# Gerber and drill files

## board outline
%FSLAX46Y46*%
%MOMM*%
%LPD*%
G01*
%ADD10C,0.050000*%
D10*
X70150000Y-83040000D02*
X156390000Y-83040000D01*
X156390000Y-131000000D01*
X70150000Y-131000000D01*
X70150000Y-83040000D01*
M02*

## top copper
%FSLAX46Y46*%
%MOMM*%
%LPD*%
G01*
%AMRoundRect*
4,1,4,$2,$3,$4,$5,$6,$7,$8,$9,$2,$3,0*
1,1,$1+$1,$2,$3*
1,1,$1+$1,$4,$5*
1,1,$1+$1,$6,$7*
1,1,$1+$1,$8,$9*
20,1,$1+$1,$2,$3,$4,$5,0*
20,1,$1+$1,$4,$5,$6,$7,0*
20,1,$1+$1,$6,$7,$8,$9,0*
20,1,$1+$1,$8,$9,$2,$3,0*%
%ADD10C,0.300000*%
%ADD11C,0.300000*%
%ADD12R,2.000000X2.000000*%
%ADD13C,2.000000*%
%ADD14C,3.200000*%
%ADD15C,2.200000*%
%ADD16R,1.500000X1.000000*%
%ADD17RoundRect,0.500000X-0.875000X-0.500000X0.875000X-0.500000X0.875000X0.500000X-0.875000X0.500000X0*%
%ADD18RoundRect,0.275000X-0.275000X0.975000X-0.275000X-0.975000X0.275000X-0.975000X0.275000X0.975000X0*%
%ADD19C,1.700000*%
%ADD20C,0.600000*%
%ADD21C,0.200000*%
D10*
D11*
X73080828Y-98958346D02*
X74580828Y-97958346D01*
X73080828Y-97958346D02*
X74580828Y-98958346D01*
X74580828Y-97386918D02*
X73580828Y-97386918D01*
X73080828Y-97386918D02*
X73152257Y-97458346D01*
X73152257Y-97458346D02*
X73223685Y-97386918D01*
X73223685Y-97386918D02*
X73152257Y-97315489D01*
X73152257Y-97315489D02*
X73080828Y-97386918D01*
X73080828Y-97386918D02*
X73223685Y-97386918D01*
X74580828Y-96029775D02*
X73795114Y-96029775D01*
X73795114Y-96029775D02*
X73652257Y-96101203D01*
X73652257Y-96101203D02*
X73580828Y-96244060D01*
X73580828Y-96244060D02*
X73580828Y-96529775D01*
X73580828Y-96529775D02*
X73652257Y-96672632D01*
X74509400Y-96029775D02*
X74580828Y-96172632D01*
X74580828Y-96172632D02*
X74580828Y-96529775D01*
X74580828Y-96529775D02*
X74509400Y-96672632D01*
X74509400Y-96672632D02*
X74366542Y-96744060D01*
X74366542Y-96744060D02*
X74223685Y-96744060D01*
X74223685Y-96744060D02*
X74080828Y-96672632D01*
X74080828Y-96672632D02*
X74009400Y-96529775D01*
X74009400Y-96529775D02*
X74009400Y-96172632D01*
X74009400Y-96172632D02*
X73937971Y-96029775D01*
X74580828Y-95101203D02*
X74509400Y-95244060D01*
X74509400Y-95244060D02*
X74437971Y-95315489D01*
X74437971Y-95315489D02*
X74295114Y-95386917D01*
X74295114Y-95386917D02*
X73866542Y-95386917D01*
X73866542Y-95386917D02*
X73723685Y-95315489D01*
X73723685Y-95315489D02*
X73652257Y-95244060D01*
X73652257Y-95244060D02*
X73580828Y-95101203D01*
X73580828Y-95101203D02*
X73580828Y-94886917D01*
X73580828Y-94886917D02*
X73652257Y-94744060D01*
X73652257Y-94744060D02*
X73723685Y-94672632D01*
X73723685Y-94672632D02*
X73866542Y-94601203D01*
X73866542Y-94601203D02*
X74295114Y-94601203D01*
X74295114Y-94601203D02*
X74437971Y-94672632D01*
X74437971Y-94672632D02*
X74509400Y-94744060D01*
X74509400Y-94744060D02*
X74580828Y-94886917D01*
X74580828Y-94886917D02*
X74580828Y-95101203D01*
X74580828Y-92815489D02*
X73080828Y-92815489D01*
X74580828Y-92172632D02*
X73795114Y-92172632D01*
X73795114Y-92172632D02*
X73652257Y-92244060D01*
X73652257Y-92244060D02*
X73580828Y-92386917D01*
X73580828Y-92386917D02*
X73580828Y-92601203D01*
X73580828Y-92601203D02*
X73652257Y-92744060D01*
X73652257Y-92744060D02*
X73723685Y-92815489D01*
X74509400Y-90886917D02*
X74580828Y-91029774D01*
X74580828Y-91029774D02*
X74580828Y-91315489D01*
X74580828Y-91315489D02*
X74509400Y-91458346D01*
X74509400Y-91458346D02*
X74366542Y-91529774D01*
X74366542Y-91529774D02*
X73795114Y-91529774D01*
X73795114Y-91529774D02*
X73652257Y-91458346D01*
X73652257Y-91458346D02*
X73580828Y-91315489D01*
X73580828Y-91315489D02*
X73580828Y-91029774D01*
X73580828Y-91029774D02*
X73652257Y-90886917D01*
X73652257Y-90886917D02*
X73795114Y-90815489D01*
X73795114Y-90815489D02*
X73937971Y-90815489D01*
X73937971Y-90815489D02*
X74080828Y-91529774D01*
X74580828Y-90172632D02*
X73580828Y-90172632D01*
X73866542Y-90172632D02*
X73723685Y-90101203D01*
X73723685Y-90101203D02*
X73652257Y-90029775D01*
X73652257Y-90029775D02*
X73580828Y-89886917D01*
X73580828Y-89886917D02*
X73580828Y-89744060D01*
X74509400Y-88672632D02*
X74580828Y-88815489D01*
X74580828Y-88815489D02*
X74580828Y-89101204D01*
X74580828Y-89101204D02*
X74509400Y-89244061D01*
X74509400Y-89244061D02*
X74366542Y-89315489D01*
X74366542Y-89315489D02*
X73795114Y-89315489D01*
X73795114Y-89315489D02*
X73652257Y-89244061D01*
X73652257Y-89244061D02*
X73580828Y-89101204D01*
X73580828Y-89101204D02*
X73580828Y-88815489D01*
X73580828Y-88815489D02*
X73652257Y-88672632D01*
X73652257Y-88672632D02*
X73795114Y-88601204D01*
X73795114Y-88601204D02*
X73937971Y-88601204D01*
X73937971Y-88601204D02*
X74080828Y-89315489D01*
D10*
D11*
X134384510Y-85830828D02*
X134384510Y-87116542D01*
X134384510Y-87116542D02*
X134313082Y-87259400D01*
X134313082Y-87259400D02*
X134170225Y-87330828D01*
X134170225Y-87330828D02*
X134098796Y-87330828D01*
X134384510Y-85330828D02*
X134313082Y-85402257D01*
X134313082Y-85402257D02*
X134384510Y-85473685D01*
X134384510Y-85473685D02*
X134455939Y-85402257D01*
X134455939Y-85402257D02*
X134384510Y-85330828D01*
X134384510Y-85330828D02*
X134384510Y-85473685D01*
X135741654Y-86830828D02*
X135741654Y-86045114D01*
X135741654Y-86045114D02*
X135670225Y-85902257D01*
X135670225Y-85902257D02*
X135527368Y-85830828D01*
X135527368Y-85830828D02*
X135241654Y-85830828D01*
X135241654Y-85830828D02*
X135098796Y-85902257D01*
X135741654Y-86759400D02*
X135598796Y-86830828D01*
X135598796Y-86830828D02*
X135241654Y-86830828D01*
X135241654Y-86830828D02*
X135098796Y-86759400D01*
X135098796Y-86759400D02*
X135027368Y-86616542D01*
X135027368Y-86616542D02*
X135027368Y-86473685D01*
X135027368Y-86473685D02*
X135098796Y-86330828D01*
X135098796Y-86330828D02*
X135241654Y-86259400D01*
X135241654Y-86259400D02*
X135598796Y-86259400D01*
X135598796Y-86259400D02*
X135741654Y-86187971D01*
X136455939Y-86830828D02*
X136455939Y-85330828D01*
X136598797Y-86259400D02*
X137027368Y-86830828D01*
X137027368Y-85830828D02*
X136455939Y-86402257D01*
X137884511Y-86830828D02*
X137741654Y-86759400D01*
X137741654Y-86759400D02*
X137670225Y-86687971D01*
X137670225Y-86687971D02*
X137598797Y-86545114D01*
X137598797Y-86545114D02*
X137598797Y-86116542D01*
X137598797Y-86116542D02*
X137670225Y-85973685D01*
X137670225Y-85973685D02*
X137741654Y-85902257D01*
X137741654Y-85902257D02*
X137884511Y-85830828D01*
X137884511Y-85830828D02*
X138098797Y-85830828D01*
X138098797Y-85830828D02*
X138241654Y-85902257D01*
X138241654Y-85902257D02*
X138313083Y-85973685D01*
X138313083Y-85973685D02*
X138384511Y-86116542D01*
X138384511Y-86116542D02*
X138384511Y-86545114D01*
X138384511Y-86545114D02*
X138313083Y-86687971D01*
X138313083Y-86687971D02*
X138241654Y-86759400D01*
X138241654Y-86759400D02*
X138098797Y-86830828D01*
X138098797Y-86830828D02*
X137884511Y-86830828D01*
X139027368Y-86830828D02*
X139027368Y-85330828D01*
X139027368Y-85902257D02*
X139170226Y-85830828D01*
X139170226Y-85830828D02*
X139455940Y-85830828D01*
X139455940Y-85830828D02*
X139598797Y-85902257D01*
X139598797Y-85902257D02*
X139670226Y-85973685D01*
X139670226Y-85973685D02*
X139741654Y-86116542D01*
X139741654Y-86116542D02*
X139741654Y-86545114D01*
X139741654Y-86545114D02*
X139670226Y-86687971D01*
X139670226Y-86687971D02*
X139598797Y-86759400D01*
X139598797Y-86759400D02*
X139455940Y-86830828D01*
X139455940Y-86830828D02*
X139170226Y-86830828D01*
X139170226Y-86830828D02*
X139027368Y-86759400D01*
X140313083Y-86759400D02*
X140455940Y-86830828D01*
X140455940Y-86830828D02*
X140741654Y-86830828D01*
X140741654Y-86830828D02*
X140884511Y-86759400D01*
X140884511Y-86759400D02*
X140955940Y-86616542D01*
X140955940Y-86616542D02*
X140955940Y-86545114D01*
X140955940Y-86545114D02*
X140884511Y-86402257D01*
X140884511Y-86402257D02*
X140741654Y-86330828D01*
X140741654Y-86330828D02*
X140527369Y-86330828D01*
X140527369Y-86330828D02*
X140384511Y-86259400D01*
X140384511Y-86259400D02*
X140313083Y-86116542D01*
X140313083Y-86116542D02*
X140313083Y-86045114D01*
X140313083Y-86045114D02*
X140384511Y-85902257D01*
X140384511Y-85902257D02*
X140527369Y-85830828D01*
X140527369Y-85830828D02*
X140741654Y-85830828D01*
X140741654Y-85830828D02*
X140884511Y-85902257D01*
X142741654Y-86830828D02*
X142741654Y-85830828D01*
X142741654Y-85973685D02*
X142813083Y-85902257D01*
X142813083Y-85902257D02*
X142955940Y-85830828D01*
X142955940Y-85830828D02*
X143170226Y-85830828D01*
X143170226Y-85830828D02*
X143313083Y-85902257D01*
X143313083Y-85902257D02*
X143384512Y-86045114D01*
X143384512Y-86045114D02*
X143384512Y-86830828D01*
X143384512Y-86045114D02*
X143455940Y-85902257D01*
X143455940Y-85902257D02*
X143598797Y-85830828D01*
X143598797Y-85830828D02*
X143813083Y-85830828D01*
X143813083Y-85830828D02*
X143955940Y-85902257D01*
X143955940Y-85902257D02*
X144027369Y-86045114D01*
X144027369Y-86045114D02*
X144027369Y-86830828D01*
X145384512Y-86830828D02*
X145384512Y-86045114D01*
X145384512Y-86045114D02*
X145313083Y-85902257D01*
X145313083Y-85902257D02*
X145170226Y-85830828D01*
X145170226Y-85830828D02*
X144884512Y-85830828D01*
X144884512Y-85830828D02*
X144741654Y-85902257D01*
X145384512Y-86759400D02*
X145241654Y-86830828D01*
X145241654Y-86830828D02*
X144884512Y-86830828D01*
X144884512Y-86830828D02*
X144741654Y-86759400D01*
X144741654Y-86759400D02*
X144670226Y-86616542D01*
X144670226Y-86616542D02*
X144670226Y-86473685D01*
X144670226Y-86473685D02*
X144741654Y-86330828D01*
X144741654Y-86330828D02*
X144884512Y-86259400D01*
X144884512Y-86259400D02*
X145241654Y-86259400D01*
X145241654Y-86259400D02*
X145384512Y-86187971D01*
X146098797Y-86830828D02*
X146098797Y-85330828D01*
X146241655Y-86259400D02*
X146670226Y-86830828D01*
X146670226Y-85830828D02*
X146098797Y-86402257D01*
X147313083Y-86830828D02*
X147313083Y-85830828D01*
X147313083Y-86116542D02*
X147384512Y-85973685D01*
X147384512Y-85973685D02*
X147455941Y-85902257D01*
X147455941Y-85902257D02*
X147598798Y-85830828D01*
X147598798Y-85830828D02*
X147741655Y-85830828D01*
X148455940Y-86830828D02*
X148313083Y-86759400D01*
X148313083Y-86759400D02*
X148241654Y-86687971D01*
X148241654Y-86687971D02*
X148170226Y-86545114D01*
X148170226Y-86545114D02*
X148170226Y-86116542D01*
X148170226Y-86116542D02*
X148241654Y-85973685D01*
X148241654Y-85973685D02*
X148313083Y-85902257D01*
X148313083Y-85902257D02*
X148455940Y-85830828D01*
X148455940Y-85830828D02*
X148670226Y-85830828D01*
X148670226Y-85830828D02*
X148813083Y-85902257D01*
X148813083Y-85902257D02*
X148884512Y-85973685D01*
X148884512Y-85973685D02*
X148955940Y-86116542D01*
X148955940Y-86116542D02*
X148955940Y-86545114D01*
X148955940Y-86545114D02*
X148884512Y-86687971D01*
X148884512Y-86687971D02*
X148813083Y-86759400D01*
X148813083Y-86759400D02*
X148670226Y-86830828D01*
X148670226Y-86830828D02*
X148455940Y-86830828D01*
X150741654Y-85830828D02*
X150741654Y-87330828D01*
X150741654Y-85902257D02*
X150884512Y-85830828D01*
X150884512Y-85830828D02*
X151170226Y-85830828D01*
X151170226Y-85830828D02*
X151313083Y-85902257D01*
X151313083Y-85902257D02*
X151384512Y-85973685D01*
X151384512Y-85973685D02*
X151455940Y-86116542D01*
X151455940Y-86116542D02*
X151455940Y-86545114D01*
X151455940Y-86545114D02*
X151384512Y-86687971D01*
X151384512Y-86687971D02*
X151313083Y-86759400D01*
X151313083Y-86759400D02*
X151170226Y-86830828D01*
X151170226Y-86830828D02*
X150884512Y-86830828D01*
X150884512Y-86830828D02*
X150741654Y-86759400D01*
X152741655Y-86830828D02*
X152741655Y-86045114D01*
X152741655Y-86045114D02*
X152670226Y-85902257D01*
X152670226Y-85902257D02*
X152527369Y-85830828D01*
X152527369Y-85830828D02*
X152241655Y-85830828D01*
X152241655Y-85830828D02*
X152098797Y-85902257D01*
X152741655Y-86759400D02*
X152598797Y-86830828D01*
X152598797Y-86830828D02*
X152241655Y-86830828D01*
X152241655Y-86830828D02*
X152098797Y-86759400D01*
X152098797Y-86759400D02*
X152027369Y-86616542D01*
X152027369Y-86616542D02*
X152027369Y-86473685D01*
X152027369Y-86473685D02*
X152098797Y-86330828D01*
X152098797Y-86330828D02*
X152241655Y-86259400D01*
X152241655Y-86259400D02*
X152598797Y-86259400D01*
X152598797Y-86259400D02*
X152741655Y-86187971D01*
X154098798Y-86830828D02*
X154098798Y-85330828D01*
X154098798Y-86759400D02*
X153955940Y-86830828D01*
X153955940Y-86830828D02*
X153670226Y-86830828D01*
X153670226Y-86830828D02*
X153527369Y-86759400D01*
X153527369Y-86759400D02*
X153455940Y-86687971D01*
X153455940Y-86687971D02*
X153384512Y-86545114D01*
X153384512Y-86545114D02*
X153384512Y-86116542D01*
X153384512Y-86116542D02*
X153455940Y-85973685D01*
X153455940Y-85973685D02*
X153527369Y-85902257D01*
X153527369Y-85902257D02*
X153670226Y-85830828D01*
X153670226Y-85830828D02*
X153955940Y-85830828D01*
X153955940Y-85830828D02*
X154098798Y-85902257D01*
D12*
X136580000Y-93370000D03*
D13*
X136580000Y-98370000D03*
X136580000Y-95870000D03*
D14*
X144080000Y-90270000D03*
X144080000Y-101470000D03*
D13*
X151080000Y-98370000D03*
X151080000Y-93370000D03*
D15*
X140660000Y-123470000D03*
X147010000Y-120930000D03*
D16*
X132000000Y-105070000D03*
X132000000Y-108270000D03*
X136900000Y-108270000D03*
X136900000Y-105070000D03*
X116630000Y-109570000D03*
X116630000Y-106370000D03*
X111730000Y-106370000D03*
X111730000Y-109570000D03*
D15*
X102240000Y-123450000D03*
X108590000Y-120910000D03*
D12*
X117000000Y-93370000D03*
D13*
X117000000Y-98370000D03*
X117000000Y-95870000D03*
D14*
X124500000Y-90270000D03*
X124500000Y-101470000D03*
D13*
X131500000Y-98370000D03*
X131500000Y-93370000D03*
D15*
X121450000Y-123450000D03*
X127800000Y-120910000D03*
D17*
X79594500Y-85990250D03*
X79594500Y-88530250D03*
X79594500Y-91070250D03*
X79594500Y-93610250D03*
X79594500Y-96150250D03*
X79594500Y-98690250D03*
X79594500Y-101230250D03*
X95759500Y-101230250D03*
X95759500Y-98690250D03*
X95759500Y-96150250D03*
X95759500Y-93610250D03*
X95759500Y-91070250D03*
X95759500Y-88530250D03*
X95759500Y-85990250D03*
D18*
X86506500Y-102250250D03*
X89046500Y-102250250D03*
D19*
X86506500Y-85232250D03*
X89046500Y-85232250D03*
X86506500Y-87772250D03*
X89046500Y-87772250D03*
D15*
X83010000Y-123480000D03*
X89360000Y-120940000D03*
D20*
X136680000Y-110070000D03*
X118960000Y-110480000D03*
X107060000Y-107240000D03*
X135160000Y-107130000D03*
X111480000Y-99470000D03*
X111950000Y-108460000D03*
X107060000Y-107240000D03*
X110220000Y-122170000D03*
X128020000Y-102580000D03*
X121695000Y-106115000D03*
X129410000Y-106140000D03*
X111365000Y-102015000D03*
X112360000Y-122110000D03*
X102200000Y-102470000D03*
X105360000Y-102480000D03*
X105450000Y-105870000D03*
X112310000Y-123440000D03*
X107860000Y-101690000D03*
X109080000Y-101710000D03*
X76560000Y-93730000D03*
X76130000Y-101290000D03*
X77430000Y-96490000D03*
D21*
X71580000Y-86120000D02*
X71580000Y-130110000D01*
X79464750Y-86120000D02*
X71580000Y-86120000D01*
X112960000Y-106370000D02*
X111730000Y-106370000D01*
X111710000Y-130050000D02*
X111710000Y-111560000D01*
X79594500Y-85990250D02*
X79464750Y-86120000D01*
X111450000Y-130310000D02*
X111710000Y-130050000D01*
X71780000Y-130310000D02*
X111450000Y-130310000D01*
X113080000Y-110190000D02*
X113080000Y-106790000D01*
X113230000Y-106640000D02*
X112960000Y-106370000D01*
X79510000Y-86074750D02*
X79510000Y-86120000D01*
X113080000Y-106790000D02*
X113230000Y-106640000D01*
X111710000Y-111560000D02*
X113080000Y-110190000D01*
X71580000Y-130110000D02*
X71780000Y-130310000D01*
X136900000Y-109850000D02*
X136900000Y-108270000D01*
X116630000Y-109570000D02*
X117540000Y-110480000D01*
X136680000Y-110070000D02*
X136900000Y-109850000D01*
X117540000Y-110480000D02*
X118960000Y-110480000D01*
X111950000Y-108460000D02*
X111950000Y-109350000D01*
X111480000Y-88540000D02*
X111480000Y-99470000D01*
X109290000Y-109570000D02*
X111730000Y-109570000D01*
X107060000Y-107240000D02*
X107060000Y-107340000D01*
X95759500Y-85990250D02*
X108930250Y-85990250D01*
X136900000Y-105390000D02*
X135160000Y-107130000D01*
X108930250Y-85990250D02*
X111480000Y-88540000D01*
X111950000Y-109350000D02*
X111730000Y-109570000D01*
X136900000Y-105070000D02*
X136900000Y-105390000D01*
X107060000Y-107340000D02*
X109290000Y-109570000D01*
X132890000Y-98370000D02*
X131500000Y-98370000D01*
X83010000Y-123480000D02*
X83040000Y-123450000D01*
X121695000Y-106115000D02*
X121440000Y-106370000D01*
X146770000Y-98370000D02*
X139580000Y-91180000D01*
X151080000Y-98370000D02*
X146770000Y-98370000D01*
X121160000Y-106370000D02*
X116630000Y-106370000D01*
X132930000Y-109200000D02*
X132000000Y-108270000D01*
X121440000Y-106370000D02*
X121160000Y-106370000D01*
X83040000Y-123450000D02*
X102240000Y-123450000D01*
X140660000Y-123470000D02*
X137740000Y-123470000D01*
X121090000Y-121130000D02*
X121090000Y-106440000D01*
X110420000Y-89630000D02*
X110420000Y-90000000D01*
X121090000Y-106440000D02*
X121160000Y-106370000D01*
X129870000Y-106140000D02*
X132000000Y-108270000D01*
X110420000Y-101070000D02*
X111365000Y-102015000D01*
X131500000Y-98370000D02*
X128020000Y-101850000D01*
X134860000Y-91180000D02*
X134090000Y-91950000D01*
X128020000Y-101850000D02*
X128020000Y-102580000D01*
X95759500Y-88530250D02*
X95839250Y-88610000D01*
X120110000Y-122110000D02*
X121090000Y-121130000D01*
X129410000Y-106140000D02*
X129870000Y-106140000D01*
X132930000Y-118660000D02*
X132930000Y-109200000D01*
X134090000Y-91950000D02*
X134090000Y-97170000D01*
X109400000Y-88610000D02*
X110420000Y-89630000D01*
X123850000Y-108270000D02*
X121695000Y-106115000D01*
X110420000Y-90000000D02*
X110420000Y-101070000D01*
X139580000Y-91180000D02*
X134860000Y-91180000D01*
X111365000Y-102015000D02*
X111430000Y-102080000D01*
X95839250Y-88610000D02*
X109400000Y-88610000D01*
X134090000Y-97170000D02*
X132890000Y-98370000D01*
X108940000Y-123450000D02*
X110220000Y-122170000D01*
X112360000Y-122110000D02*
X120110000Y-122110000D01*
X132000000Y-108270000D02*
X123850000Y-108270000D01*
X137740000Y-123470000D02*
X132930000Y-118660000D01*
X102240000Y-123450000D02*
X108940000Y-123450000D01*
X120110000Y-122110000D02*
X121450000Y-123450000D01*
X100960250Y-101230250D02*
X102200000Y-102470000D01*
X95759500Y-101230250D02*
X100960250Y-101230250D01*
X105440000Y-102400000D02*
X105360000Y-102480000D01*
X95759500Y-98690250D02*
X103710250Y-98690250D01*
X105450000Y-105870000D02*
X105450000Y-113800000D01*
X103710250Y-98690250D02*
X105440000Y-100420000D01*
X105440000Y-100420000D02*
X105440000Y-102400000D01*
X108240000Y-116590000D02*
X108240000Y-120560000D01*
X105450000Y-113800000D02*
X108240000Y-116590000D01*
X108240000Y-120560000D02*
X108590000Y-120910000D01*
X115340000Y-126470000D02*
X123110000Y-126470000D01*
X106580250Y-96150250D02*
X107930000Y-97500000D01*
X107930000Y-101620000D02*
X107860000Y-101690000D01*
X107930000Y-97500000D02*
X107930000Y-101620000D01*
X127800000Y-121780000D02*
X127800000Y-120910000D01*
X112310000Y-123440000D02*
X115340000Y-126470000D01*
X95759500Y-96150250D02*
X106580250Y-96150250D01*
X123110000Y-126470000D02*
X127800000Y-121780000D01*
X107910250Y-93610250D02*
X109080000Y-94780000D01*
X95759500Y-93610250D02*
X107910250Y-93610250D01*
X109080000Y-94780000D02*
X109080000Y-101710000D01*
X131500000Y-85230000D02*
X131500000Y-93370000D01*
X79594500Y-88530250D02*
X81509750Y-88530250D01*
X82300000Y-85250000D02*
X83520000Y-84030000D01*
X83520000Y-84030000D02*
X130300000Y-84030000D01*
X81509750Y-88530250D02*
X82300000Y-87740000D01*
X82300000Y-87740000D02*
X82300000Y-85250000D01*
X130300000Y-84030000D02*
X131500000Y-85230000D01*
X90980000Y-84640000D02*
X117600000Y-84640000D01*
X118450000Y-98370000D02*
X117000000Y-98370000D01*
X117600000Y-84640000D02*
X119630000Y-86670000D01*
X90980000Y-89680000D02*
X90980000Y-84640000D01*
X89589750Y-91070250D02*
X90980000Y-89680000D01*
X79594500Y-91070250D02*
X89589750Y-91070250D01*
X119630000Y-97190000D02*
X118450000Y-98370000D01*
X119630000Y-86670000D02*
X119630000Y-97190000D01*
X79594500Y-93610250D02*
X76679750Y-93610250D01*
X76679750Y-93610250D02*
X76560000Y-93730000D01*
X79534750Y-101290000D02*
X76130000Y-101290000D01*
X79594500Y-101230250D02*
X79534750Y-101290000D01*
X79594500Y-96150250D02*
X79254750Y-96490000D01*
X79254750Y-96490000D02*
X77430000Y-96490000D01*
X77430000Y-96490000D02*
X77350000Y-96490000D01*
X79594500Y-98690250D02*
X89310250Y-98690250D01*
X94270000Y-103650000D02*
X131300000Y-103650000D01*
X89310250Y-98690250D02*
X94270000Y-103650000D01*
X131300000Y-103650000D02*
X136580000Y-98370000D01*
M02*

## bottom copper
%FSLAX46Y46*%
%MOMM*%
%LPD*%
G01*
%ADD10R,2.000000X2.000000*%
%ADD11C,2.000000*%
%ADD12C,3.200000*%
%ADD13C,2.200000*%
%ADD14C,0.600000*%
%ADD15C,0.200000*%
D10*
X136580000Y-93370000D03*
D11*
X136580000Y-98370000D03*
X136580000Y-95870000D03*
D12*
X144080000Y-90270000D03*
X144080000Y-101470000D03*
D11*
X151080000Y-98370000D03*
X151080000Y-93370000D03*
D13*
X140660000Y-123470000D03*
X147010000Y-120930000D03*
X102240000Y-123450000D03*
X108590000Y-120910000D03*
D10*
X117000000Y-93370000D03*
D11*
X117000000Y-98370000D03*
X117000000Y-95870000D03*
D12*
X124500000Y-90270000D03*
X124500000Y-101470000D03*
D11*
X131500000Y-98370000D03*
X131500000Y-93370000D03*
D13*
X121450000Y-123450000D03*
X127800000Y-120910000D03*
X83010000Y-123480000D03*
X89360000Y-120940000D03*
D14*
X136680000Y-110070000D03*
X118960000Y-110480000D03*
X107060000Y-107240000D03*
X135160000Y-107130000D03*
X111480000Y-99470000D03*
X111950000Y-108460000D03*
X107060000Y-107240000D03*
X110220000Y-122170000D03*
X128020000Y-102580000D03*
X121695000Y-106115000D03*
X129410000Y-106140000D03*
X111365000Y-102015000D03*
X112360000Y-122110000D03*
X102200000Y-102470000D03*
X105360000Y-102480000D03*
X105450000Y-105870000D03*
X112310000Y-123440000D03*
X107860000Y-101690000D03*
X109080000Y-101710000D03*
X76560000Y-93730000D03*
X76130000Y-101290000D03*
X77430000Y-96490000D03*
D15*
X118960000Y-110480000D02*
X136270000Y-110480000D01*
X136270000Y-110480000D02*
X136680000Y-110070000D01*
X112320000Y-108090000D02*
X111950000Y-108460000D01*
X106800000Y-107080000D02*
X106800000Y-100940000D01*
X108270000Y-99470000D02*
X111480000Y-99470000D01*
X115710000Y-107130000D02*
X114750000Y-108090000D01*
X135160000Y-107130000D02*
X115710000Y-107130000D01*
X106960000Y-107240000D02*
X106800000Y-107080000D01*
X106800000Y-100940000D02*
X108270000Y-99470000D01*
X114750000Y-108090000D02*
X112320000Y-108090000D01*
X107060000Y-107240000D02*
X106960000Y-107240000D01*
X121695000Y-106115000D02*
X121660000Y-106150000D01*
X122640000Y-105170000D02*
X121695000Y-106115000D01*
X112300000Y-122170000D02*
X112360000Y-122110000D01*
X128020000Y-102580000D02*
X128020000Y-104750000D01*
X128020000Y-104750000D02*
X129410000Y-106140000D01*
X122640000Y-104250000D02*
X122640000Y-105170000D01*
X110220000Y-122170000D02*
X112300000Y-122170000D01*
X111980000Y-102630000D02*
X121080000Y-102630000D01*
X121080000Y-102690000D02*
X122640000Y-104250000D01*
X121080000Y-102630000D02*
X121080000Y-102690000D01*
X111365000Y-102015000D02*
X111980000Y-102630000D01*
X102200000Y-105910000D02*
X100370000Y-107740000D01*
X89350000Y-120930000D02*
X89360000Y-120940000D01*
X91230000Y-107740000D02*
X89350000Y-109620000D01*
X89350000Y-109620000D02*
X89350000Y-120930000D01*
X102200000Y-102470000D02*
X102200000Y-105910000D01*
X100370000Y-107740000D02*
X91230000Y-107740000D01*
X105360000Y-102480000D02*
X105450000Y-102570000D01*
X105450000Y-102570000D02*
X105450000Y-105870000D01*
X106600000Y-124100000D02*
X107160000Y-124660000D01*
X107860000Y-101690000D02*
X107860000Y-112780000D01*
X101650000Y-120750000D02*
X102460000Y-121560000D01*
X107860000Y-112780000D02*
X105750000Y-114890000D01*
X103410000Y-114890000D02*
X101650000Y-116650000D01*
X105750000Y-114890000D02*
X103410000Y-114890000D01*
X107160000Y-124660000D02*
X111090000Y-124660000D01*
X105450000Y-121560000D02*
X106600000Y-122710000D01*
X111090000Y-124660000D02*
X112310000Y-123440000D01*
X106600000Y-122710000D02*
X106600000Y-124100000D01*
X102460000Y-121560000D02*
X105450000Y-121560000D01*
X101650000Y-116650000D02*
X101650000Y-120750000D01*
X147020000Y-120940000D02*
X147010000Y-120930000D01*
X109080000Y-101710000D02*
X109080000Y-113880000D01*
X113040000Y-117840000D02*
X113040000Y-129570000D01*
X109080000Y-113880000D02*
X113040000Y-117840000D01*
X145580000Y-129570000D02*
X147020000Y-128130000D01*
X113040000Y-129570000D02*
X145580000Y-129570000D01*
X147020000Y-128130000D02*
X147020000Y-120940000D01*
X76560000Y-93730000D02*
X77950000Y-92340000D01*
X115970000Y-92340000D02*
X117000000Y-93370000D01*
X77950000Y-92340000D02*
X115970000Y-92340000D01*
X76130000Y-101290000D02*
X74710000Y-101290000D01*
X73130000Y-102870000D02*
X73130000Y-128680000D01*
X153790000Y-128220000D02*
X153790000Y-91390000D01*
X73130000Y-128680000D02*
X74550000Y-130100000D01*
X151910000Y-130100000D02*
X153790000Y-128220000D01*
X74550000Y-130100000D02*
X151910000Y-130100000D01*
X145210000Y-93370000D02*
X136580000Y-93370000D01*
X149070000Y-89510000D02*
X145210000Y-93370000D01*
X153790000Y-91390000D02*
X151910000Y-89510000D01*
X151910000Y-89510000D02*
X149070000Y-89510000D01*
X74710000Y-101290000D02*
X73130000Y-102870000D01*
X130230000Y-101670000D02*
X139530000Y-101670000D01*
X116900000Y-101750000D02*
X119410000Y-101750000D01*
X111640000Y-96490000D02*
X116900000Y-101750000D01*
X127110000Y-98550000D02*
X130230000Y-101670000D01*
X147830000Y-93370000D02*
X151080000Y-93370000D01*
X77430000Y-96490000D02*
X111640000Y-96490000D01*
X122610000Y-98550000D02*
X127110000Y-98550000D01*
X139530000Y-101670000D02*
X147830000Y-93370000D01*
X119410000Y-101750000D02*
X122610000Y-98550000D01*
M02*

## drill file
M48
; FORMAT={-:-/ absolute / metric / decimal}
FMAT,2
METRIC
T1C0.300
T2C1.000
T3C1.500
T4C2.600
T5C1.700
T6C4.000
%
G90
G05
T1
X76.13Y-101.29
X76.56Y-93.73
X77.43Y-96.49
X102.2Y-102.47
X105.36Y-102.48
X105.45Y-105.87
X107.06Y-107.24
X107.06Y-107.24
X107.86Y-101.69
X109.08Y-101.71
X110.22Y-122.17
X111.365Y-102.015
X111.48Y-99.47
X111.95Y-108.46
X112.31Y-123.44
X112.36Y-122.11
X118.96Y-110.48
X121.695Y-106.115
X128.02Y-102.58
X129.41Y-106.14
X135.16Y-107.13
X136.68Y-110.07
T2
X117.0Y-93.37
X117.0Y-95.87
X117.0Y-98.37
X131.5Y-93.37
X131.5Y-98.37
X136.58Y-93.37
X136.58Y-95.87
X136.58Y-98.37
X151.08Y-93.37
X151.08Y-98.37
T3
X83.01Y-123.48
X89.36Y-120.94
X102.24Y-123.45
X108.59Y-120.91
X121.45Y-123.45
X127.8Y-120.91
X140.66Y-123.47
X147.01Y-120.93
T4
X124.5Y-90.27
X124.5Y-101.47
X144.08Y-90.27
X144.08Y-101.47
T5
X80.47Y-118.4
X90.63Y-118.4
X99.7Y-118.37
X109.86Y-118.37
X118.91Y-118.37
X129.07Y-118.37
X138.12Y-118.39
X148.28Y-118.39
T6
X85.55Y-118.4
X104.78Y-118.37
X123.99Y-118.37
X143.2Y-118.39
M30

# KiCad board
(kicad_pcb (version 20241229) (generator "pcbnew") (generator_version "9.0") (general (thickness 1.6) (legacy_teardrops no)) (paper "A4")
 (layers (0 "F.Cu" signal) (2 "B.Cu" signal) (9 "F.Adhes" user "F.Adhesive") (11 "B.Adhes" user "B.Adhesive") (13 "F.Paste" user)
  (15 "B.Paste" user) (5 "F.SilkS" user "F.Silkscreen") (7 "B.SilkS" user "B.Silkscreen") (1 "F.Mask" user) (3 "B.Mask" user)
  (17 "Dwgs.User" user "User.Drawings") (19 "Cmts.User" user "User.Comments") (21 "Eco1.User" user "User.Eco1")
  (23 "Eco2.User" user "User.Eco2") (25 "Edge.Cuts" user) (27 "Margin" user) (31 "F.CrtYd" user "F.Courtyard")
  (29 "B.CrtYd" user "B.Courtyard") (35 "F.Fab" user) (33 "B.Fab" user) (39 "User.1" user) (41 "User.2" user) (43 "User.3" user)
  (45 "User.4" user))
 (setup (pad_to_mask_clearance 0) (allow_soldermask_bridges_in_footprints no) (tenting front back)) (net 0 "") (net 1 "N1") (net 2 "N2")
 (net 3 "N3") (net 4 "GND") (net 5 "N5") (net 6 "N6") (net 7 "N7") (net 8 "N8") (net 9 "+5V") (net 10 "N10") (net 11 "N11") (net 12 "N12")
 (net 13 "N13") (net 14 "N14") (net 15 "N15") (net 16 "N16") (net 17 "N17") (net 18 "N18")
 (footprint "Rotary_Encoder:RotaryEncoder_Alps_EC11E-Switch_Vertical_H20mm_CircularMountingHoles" (layer "F.Cu") (at 136.58 93.37)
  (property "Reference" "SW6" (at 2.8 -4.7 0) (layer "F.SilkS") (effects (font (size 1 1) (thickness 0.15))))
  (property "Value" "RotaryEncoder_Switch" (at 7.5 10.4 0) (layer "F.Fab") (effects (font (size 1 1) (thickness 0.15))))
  (pad "A" thru_hole rect (at 0 0) (size 2 2) (drill 1) (layers "*.Cu" "*.Mask") (remove_unused_layers no) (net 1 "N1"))
  (pad "B" thru_hole circle (at 0 5) (size 2 2) (drill 1) (layers "*.Cu" "*.Mask") (remove_unused_layers no) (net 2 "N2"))
  (pad "C" thru_hole circle (at 0 2.5) (size 2 2) (drill 1) (layers "*.Cu" "*.Mask") (remove_unused_layers no) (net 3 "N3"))
  (pad "MP" thru_hole circle (at 7.5 -3.1) (size 3.2 3.2) (drill 2.6) (layers "*.Cu" "*.Mask") (remove_unused_layers no))
  (pad "MP" thru_hole circle (at 7.5 8.1) (size 3.2 3.2) (drill 2.6) (layers "*.Cu" "*.Mask") (remove_unused_layers no))
  (pad "S1" thru_hole circle (at 14.5 5) (size 2 2) (drill 1) (layers "*.Cu" "*.Mask") (remove_unused_layers no) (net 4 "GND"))
  (pad "S2" thru_hole circle (at 14.5 0) (size 2 2) (drill 1) (layers "*.Cu" "*.Mask") (remove_unused_layers no) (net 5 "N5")))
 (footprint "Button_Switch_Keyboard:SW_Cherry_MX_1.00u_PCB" (layer "F.Cu") (at 140.66 123.47 180)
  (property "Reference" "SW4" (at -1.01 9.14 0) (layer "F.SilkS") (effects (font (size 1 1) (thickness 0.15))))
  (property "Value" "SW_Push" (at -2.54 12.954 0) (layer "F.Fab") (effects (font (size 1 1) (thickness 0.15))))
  (pad "" np_thru_hole circle (at -7.62 5.08 180) (size 1.7 1.7) (drill 1.7) (layers "*.Cu" "*.Mask"))
  (pad "" np_thru_hole circle (at -2.54 5.08 180) (size 4 4) (drill 4) (layers "*.Cu" "*.Mask"))
  (pad "" np_thru_hole circle (at 2.54 5.08 180) (size 1.7 1.7) (drill 1.7) (layers "*.Cu" "*.Mask"))
  (pad "1" thru_hole circle (at 0 0 180) (size 2.2 2.2) (drill 1.5) (layers "*.Cu" "*.Mask") (remove_unused_layers no) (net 4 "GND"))
  (pad "2" thru_hole circle (at -6.35 2.54 180) (size 2.2 2.2) (drill 1.5) (layers "*.Cu" "*.Mask") (remove_unused_layers no) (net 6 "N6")))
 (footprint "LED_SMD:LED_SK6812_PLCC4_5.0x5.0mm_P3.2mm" (layer "F.Cu") (at 134.45 106.67)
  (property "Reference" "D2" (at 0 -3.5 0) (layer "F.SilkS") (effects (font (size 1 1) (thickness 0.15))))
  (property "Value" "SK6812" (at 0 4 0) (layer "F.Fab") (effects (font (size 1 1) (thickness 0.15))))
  (pad "1" smd rect (at -2.45 -1.6 180) (size 1.5 1) (layers "F.Cu" "F.Mask" "F.Paste") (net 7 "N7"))
  (pad "2" smd rect (at -2.45 1.6 180) (size 1.5 1) (layers "F.Cu" "F.Mask" "F.Paste") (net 4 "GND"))
  (pad "3" smd rect (at 2.45 1.6 180) (size 1.5 1) (layers "F.Cu" "F.Mask" "F.Paste") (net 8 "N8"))
  (pad "4" smd rect (at 2.45 -1.6 180) (size 1.5 1) (layers "F.Cu" "F.Mask" "F.Paste") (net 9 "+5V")))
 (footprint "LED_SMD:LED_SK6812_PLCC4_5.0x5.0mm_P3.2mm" (layer "F.Cu") (at 114.18 107.97 180)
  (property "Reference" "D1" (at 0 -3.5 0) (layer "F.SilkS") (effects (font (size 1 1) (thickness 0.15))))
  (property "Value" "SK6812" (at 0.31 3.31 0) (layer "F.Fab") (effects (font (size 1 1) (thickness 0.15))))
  (pad "1" smd rect (at -2.45 -1.6) (size 1.5 1) (layers "F.Cu" "F.Mask" "F.Paste") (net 8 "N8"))
  (pad "2" smd rect (at -2.45 1.6) (size 1.5 1) (layers "F.Cu" "F.Mask" "F.Paste") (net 4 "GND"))
  (pad "3" smd rect (at 2.45 1.6) (size 1.5 1) (layers "F.Cu" "F.Mask" "F.Paste") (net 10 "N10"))
  (pad "4" smd rect (at 2.45 -1.6) (size 1.5 1) (layers "F.Cu" "F.Mask" "F.Paste") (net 9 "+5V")))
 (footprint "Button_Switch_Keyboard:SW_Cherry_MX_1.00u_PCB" (layer "F.Cu") (at 102.24 123.45 180)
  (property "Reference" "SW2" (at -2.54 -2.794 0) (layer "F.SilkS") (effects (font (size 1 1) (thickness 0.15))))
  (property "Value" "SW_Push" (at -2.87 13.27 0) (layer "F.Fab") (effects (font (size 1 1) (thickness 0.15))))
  (pad "" np_thru_hole circle (at -7.62 5.08 180) (size 1.7 1.7) (drill 1.7) (layers "*.Cu" "*.Mask"))
  (pad "" np_thru_hole circle (at -2.54 5.08 180) (size 4 4) (drill 4) (layers "*.Cu" "*.Mask"))
  (pad "" np_thru_hole circle (at 2.54 5.08 180) (size 1.7 1.7) (drill 1.7) (layers "*.Cu" "*.Mask"))
  (pad "1" thru_hole circle (at 0 0 180) (size 2.2 2.2) (drill 1.5) (layers "*.Cu" "*.Mask") (remove_unused_layers no) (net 4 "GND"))
  (pad "2" thru_hole circle (at -6.35 2.54 180) (size 2.2 2.2) (drill 1.5) (layers "*.Cu" "*.Mask") (remove_unused_layers no) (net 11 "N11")))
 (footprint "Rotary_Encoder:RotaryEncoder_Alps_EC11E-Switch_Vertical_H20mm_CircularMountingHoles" (layer "F.Cu") (at 117 93.37)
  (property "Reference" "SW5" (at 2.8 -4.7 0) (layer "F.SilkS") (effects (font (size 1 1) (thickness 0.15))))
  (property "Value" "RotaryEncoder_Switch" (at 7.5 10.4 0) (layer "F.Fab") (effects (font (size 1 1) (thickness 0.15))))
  (pad "A" thru_hole rect (at 0 0) (size 2 2) (drill 1) (layers "*.Cu" "*.Mask") (remove_unused_layers no) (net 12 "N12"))
  (pad "B" thru_hole circle (at 0 5) (size 2 2) (drill 1) (layers "*.Cu" "*.Mask") (remove_unused_layers no) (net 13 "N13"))
  (pad "C" thru_hole circle (at 0 2.5) (size 2 2) (drill 1) (layers "*.Cu" "*.Mask") (remove_unused_layers no) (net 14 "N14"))
  (pad "MP" thru_hole circle (at 7.5 -3.1) (size 3.2 3.2) (drill 2.6) (layers "*.Cu" "*.Mask") (remove_unused_layers no))
  (pad "MP" thru_hole circle (at 7.5 8.1) (size 3.2 3.2) (drill 2.6) (layers "*.Cu" "*.Mask") (remove_unused_layers no))
  (pad "S1" thru_hole circle (at 14.5 5) (size 2 2) (drill 1) (layers "*.Cu" "*.Mask") (remove_unused_layers no) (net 4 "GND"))
  (pad "S2" thru_hole circle (at 14.5 0) (size 2 2) (drill 1) (layers "*.Cu" "*.Mask") (remove_unused_layers no) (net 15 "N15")))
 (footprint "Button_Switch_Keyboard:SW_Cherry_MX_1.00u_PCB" (layer "F.Cu") (at 121.45 123.45 180)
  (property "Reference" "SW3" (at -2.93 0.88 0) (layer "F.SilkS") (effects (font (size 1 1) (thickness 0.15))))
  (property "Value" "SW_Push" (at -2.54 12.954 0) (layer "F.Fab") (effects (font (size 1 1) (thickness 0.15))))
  (pad "" np_thru_hole circle (at -7.62 5.08 180) (size 1.7 1.7) (drill 1.7) (layers "*.Cu" "*.Mask"))
  (pad "" np_thru_hole circle (at -2.54 5.08 180) (size 4 4) (drill 4) (layers "*.Cu" "*.Mask"))
  (pad "" np_thru_hole circle (at 2.54 5.08 180) (size 1.7 1.7) (drill 1.7) (layers "*.Cu" "*.Mask"))
  (pad "1" thru_hole circle (at 0 0 180) (size 2.2 2.2) (drill 1.5) (layers "*.Cu" "*.Mask") (remove_unused_layers no) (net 4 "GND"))
  (pad "2" thru_hole circle (at -6.35 2.54 180) (size 2.2 2.2) (drill 1.5) (layers "*.Cu" "*.Mask") (remove_unused_layers no) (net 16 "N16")))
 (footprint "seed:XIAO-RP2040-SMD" (layer "F.Cu") (at 87.5945 93.61025)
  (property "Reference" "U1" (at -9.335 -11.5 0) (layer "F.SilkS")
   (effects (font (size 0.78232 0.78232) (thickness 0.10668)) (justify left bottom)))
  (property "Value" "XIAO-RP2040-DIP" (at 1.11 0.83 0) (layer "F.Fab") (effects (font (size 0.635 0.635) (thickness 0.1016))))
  (pad "1" smd roundrect (at -8 -7.62) (size 2.75 2) (layers "F.Cu" "F.Mask" "F.Paste") (roundrect_rratio 0.25) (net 10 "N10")
   (solder_mask_margin 0.0508) (thermal_bridge_angle 45))
  (pad "2" smd roundrect (at -8 -5.08) (size 2.75 2) (layers "F.Cu" "F.Mask" "F.Paste") (roundrect_rratio 0.25) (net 15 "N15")
   (solder_mask_margin 0.0508) (thermal_bridge_angle 45))
  (pad "3" smd roundrect (at -8 -2.54) (size 2.75 2) (layers "F.Cu" "F.Mask" "F.Paste") (roundrect_rratio 0.25) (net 13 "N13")
   (solder_mask_margin 0.0508) (thermal_bridge_angle 45))
  (pad "4" smd roundrect (at -8 0) (size 2.75 2) (layers "F.Cu" "F.Mask" "F.Paste") (roundrect_rratio 0.25) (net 12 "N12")
   (solder_mask_margin 0.0508) (thermal_bridge_angle 45))
  (pad "5" smd roundrect (at -8 2.54) (size 2.75 2) (layers "F.Cu" "F.Mask" "F.Paste") (roundrect_rratio 0.25) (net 5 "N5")
   (solder_mask_margin 0.0508) (thermal_bridge_angle 45))
  (pad "6" smd roundrect (at -8 5.08) (size 2.75 2) (layers "F.Cu" "F.Mask" "F.Paste") (roundrect_rratio 0.25) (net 2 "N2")
   (solder_mask_margin 0.0508) (thermal_bridge_angle 45))
  (pad "7" smd roundrect (at -8 7.62) (size 2.75 2) (layers "F.Cu" "F.Mask" "F.Paste") (roundrect_rratio 0.25) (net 1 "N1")
   (solder_mask_margin 0.0508) (thermal_bridge_angle 45))
  (pad "8" smd roundrect (at 8.165 7.62) (size 2.75 2) (layers "F.Cu" "F.Mask" "F.Paste") (roundrect_rratio 0.25) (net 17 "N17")
   (solder_mask_margin 0.0508) (thermal_bridge_angle 45))
  (pad "9" smd roundrect (at 8.165 5.08) (size 2.75 2) (layers "F.Cu" "F.Mask" "F.Paste") (roundrect_rratio 0.25) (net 11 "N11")
   (solder_mask_margin 0.0508) (thermal_bridge_angle 45))
  (pad "10" smd roundrect (at 8.165 2.54) (size 2.75 2) (layers "F.Cu" "F.Mask" "F.Paste") (roundrect_rratio 0.25) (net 16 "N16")
   (solder_mask_margin 0.0508) (thermal_bridge_angle 45))
  (pad "11" smd roundrect (at 8.165 0) (size 2.75 2) (layers "F.Cu" "F.Mask" "F.Paste") (roundrect_rratio 0.25) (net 6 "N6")
   (solder_mask_margin 0.0508) (thermal_bridge_angle 45))
  (pad "12" smd roundrect (at 8.165 -2.54) (size 2.75 2) (layers "F.Cu" "F.Mask" "F.Paste") (roundrect_rratio 0.25) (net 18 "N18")
   (solder_mask_margin 0.0508) (thermal_bridge_angle 45))
  (pad "13" smd roundrect (at 8.165 -5.08) (size 2.75 2) (layers "F.Cu" "F.Mask" "F.Paste") (roundrect_rratio 0.25) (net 4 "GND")
   (solder_mask_margin 0.0508) (thermal_bridge_angle 45))
  (pad "14" smd roundrect (at 8.165 -7.62) (size 2.75 2) (layers "F.Cu" "F.Mask" "F.Paste") (roundrect_rratio 0.25) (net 9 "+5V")
   (solder_mask_margin 0.0508) (thermal_bridge_angle 45))
  (pad "15" smd roundrect (at -1.088 8.64 270) (size 2.5 1.1) (layers "F.Cu" "F.Mask" "F.Paste") (roundrect_rratio 0.25)
   (thermal_bridge_angle 45))
  (pad "16" smd roundrect (at 1.452 8.64 270) (size 2.5 1.1) (layers "F.Cu" "F.Mask" "F.Paste") (roundrect_rratio 0.25)
   (thermal_bridge_angle 45))
  (pad "17" smd circle (at -1.088 -8.378) (size 1.7 1.7) (layers "F.Cu" "F.Mask" "F.Paste"))
  (pad "18" smd circle (at 1.452 -8.378) (size 1.7 1.7) (layers "F.Cu" "F.Mask" "F.Paste"))
  (pad "19" smd circle (at -1.088 -5.838) (size 1.7 1.7) (layers "F.Cu" "F.Mask" "F.Paste"))
  (pad "20" smd circle (at 1.452 -5.838) (size 1.7 1.7) (layers "F.Cu" "F.Mask" "F.Paste")))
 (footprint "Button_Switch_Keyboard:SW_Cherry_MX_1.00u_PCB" (layer "F.Cu") (at 83.01 123.48 180)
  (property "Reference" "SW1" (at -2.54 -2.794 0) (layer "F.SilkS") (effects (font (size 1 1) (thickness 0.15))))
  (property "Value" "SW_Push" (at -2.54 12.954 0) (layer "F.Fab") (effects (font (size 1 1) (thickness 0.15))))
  (pad "" np_thru_hole circle (at -7.62 5.08 180) (size 1.7 1.7) (drill 1.7) (layers "*.Cu" "*.Mask"))
  (pad "" np_thru_hole circle (at -2.54 5.08 180) (size 4 4) (drill 4) (layers "*.Cu" "*.Mask"))
  (pad "" np_thru_hole circle (at 2.54 5.08 180) (size 1.7 1.7) (drill 1.7) (layers "*.Cu" "*.Mask"))
  (pad "1" thru_hole circle (at 0 0 180) (size 2.2 2.2) (drill 1.5) (layers "*.Cu" "*.Mask") (remove_unused_layers no) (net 4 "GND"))
  (pad "2" thru_hole circle (at -6.35 2.54 180) (size 2.2 2.2) (drill 1.5) (layers "*.Cu" "*.Mask") (remove_unused_layers no) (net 17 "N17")))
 (gr_rect (start 70.15 83.04) (end 156.39 131) (stroke (width 0.05) (type default)) (fill no) (layer "Edge.Cuts"))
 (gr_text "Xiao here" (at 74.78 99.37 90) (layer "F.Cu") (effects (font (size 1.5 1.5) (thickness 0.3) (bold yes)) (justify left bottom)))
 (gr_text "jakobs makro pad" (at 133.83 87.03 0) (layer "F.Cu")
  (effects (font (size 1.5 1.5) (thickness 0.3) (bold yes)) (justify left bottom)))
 (segment (start 71.58 86.12) (end 71.58 130.11) (width 0.2) (layer "F.Cu") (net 10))
 (segment (start 79.46475 86.12) (end 71.58 86.12) (width 0.2) (layer "F.Cu") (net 10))
 (segment (start 112.96 106.37) (end 111.73 106.37) (width 0.2) (layer "F.Cu") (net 10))
 (segment (start 111.71 130.05) (end 111.71 111.56) (width 0.2) (layer "F.Cu") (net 10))
 (segment (start 79.5945 85.99025) (end 79.46475 86.12) (width 0.2) (layer "F.Cu") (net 10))
 (segment (start 111.45 130.31) (end 111.71 130.05) (width 0.2) (layer "F.Cu") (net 10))
 (segment (start 71.78 130.31) (end 111.45 130.31) (width 0.2) (layer "F.Cu") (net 10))
 (segment (start 113.08 110.19) (end 113.08 106.79) (width 0.2) (layer "F.Cu") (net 10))
 (segment (start 113.23 106.64) (end 112.96 106.37) (width 0.2) (layer "F.Cu") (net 10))
 (segment (start 79.51 86.07475) (end 79.51 86.12) (width 0.2) (layer "F.Cu") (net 10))
 (segment (start 113.08 106.79) (end 113.23 106.64) (width 0.2) (layer "F.Cu") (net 10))
 (segment (start 111.71 111.56) (end 113.08 110.19) (width 0.2) (layer "F.Cu") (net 10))
 (segment (start 71.58 130.11) (end 71.78 130.31) (width 0.2) (layer "F.Cu") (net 10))
 (segment (start 136.9 109.85) (end 136.9 108.27) (width 0.2) (layer "F.Cu") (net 8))
 (segment (start 116.63 109.57) (end 117.54 110.48) (width 0.2) (layer "F.Cu") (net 8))
 (segment (start 136.68 110.07) (end 136.9 109.85) (width 0.2) (layer "F.Cu") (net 8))
 (segment (start 117.54 110.48) (end 118.96 110.48) (width 0.2) (layer "F.Cu") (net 8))
 (via (at 136.68 110.07) (size 0.6) (drill 0.3) (layers "F.Cu" "B.Cu") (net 8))
 (via (at 118.96 110.48) (size 0.6) (drill 0.3) (layers "F.Cu" "B.Cu") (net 8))
 (segment (start 118.96 110.48) (end 136.27 110.48) (width 0.2) (layer "B.Cu") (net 8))
 (segment (start 136.27 110.48) (end 136.68 110.07) (width 0.2) (layer "B.Cu") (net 8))
 (segment (start 111.95 108.46) (end 111.95 109.35) (width 0.2) (layer "F.Cu") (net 9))
 (segment (start 111.48 88.54) (end 111.48 99.47) (width 0.2) (layer "F.Cu") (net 9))
 (segment (start 109.29 109.57) (end 111.73 109.57) (width 0.2) (layer "F.Cu") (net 9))
 (segment (start 107.06 107.24) (end 107.06 107.34) (width 0.2) (layer "F.Cu") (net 9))
 (segment (start 95.7595 85.99025) (end 108.93025 85.99025) (width 0.2) (layer "F.Cu") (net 9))
 (segment (start 136.9 105.39) (end 135.16 107.13) (width 0.2) (layer "F.Cu") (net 9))
 (segment (start 108.93025 85.99025) (end 111.48 88.54) (width 0.2) (layer "F.Cu") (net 9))
 (segment (start 111.95 109.35) (end 111.73 109.57) (width 0.2) (layer "F.Cu") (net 9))
 (segment (start 136.9 105.07) (end 136.9 105.39) (width 0.2) (layer "F.Cu") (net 9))
 (segment (start 107.06 107.34) (end 109.29 109.57) (width 0.2) (layer "F.Cu") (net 9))
 (via (at 107.06 107.24) (size 0.6) (drill 0.3) (layers "F.Cu" "B.Cu") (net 9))
 (via (at 135.16 107.13) (size 0.6) (drill 0.3) (layers "F.Cu" "B.Cu") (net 9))
 (via (at 111.48 99.47) (size 0.6) (drill 0.3) (layers "F.Cu" "B.Cu") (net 9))
 (via (at 111.95 108.46) (size 0.6) (drill 0.3) (layers "F.Cu" "B.Cu") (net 9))
 (via (at 107.06 107.24) (size 0.6) (drill 0.3) (layers "F.Cu" "B.Cu") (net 9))
 (segment (start 112.32 108.09) (end 111.95 108.46) (width 0.2) (layer "B.Cu") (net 9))
 (segment (start 106.8 107.08) (end 106.8 100.94) (width 0.2) (layer "B.Cu") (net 9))
 (segment (start 108.27 99.47) (end 111.48 99.47) (width 0.2) (layer "B.Cu") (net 9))
 (segment (start 115.71 107.13) (end 114.75 108.09) (width 0.2) (layer "B.Cu") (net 9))
 (segment (start 135.16 107.13) (end 115.71 107.13) (width 0.2) (layer "B.Cu") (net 9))
 (segment (start 106.96 107.24) (end 106.8 107.08) (width 0.2) (layer "B.Cu") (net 9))
 (segment (start 106.8 100.94) (end 108.27 99.47) (width 0.2) (layer "B.Cu") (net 9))
 (segment (start 114.75 108.09) (end 112.32 108.09) (width 0.2) (layer "B.Cu") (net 9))
 (segment (start 107.06 107.24) (end 106.96 107.24) (width 0.2) (layer "B.Cu") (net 9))
 (segment (start 132.89 98.37) (end 131.5 98.37) (width 0.2) (layer "F.Cu") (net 4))
 (segment (start 83.01 123.48) (end 83.04 123.45) (width 0.2) (layer "F.Cu") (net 4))
 (segment (start 121.695 106.115) (end 121.44 106.37) (width 0.2) (layer "F.Cu") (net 4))
 (segment (start 146.77 98.37) (end 139.58 91.18) (width 0.2) (layer "F.Cu") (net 4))
 (segment (start 151.08 98.37) (end 146.77 98.37) (width 0.2) (layer "F.Cu") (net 4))
 (segment (start 121.16 106.37) (end 116.63 106.37) (width 0.2) (layer "F.Cu") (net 4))
 (segment (start 132.93 109.2) (end 132 108.27) (width 0.2) (layer "F.Cu") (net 4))
 (segment (start 121.44 106.37) (end 121.16 106.37) (width 0.2) (layer "F.Cu") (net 4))
 (segment (start 83.04 123.45) (end 102.24 123.45) (width 0.2) (layer "F.Cu") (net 4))
 (segment (start 140.66 123.47) (end 137.74 123.47) (width 0.2) (layer "F.Cu") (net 4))
 (segment (start 121.09 121.13) (end 121.09 106.44) (width 0.2) (layer "F.Cu") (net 4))
 (segment (start 110.42 89.63) (end 110.42 90) (width 0.2) (layer "F.Cu") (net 4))
 (segment (start 121.09 106.44) (end 121.16 106.37) (width 0.2) (layer "F.Cu") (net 4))
 (segment (start 129.87 106.14) (end 132 108.27) (width 0.2) (layer "F.Cu") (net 4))
 (segment (start 110.42 101.07) (end 111.365 102.015) (width 0.2) (layer "F.Cu") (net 4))
 (segment (start 131.5 98.37) (end 128.02 101.85) (width 0.2) (layer "F.Cu") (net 4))
 (segment (start 134.86 91.18) (end 134.09 91.95) (width 0.2) (layer "F.Cu") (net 4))
 (segment (start 128.02 101.85) (end 128.02 102.58) (width 0.2) (layer "F.Cu") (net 4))
 (segment (start 95.7595 88.53025) (end 95.83925 88.61) (width 0.2) (layer "F.Cu") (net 4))
 (segment (start 120.11 122.11) (end 121.09 121.13) (width 0.2) (layer "F.Cu") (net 4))
 (segment (start 129.41 106.14) (end 129.87 106.14) (width 0.2) (layer "F.Cu") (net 4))
 (segment (start 132.93 118.66) (end 132.93 109.2) (width 0.2) (layer "F.Cu") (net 4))
 (segment (start 134.09 91.95) (end 134.09 97.17) (width 0.2) (layer "F.Cu") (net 4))
 (segment (start 109.4 88.61) (end 110.42 89.63) (width 0.2) (layer "F.Cu") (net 4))
 (segment (start 123.85 108.27) (end 121.695 106.115) (width 0.2) (layer "F.Cu") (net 4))
 (segment (start 110.42 90) (end 110.42 101.07) (width 0.2) (layer "F.Cu") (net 4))
 (segment (start 139.58 91.18) (end 134.86 91.18) (width 0.2) (layer "F.Cu") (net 4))
 (segment (start 111.365 102.015) (end 111.43 102.08) (width 0.2) (layer "F.Cu") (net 4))
 (segment (start 95.83925 88.61) (end 109.4 88.61) (width 0.2) (layer "F.Cu") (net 4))
 (segment (start 134.09 97.17) (end 132.89 98.37) (width 0.2) (layer "F.Cu") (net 4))
 (segment (start 108.94 123.45) (end 110.22 122.17) (width 0.2) (layer "F.Cu") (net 4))
 (segment (start 112.36 122.11) (end 120.11 122.11) (width 0.2) (layer "F.Cu") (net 4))
 (segment (start 132 108.27) (end 123.85 108.27) (width 0.2) (layer "F.Cu") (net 4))
 (segment (start 137.74 123.47) (end 132.93 118.66) (width 0.2) (layer "F.Cu") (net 4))
 (segment (start 102.24 123.45) (end 108.94 123.45) (width 0.2) (layer "F.Cu") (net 4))
 (segment (start 120.11 122.11) (end 121.45 123.45) (width 0.2) (layer "F.Cu") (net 4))
 (via (at 110.22 122.17) (size 0.6) (drill 0.3) (layers "F.Cu" "B.Cu") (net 4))
 (via (at 128.02 102.58) (size 0.6) (drill 0.3) (layers "F.Cu" "B.Cu") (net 4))
 (via (at 121.695 106.115) (size 0.6) (drill 0.3) (layers "F.Cu" "B.Cu") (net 4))
 (via (at 129.41 106.14) (size 0.6) (drill 0.3) (layers "F.Cu" "B.Cu") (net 4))
 (via (at 111.365 102.015) (size 0.6) (drill 0.3) (layers "F.Cu" "B.Cu") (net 4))
 (via (at 112.36 122.11) (size 0.6) (drill 0.3) (layers "F.Cu" "B.Cu") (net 4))
 (segment (start 121.695 106.115) (end 121.66 106.15) (width 0.2) (layer "B.Cu") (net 4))
 (segment (start 122.64 105.17) (end 121.695 106.115) (width 0.2) (layer "B.Cu") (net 4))
 (segment (start 112.3 122.17) (end 112.36 122.11) (width 0.2) (layer "B.Cu") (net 4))
 (segment (start 128.02 102.58) (end 128.02 104.75) (width 0.2) (layer "B.Cu") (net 4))
 (segment (start 128.02 104.75) (end 129.41 106.14) (width 0.2) (layer "B.Cu") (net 4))
 (segment (start 122.64 104.25) (end 122.64 105.17) (width 0.2) (layer "B.Cu") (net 4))
 (segment (start 110.22 122.17) (end 112.3 122.17) (width 0.2) (layer "B.Cu") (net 4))
 (segment (start 111.98 102.63) (end 121.08 102.63) (width 0.2) (layer "B.Cu") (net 4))
 (segment (start 121.08 102.69) (end 122.64 104.25) (width 0.2) (layer "B.Cu") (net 4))
 (segment (start 121.08 102.63) (end 121.08 102.69) (width 0.2) (layer "B.Cu") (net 4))
 (segment (start 111.365 102.015) (end 111.98 102.63) (width 0.2) (layer "B.Cu") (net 4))
 (segment (start 100.96025 101.23025) (end 102.2 102.47) (width 0.2) (layer "F.Cu") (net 17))
 (segment (start 95.7595 101.23025) (end 100.96025 101.23025) (width 0.2) (layer "F.Cu") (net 17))
 (via (at 102.2 102.47) (size 0.6) (drill 0.3) (layers "F.Cu" "B.Cu") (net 17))
 (segment (start 102.2 105.91) (end 100.37 107.74) (width 0.2) (layer "B.Cu") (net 17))
 (segment (start 89.35 120.93) (end 89.36 120.94) (width 0.2) (layer "B.Cu") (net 17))
 (segment (start 91.23 107.74) (end 89.35 109.62) (width 0.2) (layer "B.Cu") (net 17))
 (segment (start 89.35 109.62) (end 89.35 120.93) (width 0.2) (layer "B.Cu") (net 17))
 (segment (start 102.2 102.47) (end 102.2 105.91) (width 0.2) (layer "B.Cu") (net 17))
 (segment (start 100.37 107.74) (end 91.23 107.74) (width 0.2) (layer "B.Cu") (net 17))
 (segment (start 105.44 102.4) (end 105.36 102.48) (width 0.2) (layer "F.Cu") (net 11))
 (segment (start 95.7595 98.69025) (end 103.71025 98.69025) (width 0.2) (layer "F.Cu") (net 11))
 (segment (start 105.45 105.87) (end 105.45 113.8) (width 0.2) (layer "F.Cu") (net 11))
 (segment (start 103.71025 98.69025) (end 105.44 100.42) (width 0.2) (layer "F.Cu") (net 11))
 (segment (start 105.44 100.42) (end 105.44 102.4) (width 0.2) (layer "F.Cu") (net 11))
 (segment (start 108.24 116.59) (end 108.24 120.56) (width 0.2) (layer "F.Cu") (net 11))
 (segment (start 105.45 113.8) (end 108.24 116.59) (width 0.2) (layer "F.Cu") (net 11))
 (segment (start 108.24 120.56) (end 108.59 120.91) (width 0.2) (layer "F.Cu") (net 11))
 (via (at 105.36 102.48) (size 0.6) (drill 0.3) (layers "F.Cu" "B.Cu") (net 11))
 (via (at 105.45 105.87) (size 0.6) (drill 0.3) (layers "F.Cu" "B.Cu") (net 11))
 (segment (start 105.36 102.48) (end 105.45 102.57) (width 0.2) (layer "B.Cu") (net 11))
 (segment (start 105.45 102.57) (end 105.45 105.87) (width 0.2) (layer "B.Cu") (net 11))
 (segment (start 115.34 126.47) (end 123.11 126.47) (width 0.2) (layer "F.Cu") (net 16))
 (segment (start 106.58025 96.15025) (end 107.93 97.5) (width 0.2) (layer "F.Cu") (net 16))
 (segment (start 107.93 101.62) (end 107.86 101.69) (width 0.2) (layer "F.Cu") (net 16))
 (segment (start 107.93 97.5) (end 107.93 101.62) (width 0.2) (layer "F.Cu") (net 16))
 (segment (start 127.8 121.78) (end 127.8 120.91) (width 0.2) (layer "F.Cu") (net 16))
 (segment (start 112.31 123.44) (end 115.34 126.47) (width 0.2) (layer "F.Cu") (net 16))
 (segment (start 95.7595 96.15025) (end 106.58025 96.15025) (width 0.2) (layer "F.Cu") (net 16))
 (segment (start 123.11 126.47) (end 127.8 121.78) (width 0.2) (layer "F.Cu") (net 16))
 (via (at 112.31 123.44) (size 0.6) (drill 0.3) (layers "F.Cu" "B.Cu") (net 16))
 (via (at 107.86 101.69) (size 0.6) (drill 0.3) (layers "F.Cu" "B.Cu") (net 16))
 (segment (start 106.6 124.1) (end 107.16 124.66) (width 0.2) (layer "B.Cu") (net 16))
 (segment (start 107.86 101.69) (end 107.86 112.78) (width 0.2) (layer "B.Cu") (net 16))
 (segment (start 101.65 120.75) (end 102.46 121.56) (width 0.2) (layer "B.Cu") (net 16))
 (segment (start 107.86 112.78) (end 105.75 114.89) (width 0.2) (layer "B.Cu") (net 16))
 (segment (start 103.41 114.89) (end 101.65 116.65) (width 0.2) (layer "B.Cu") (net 16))
 (segment (start 105.75 114.89) (end 103.41 114.89) (width 0.2) (layer "B.Cu") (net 16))
 (segment (start 107.16 124.66) (end 111.09 124.66) (width 0.2) (layer "B.Cu") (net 16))
 (segment (start 105.45 121.56) (end 106.6 122.71) (width 0.2) (layer "B.Cu") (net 16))
 (segment (start 111.09 124.66) (end 112.31 123.44) (width 0.2) (layer "B.Cu") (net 16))
 (segment (start 106.6 122.71) (end 106.6 124.1) (width 0.2) (layer "B.Cu") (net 16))
 (segment (start 102.46 121.56) (end 105.45 121.56) (width 0.2) (layer "B.Cu") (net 16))
 (segment (start 101.65 116.65) (end 101.65 120.75) (width 0.2) (layer "B.Cu") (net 16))
 (segment (start 107.91025 93.61025) (end 109.08 94.78) (width 0.2) (layer "F.Cu") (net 6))
 (segment (start 95.7595 93.61025) (end 107.91025 93.61025) (width 0.2) (layer "F.Cu") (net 6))
 (segment (start 109.08 94.78) (end 109.08 101.71) (width 0.2) (layer "F.Cu") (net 6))
 (via (at 109.08 101.71) (size 0.6) (drill 0.3) (layers "F.Cu" "B.Cu") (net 6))
 (segment (start 147.02 120.94) (end 147.01 120.93) (width 0.2) (layer "B.Cu") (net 6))
 (segment (start 109.08 101.71) (end 109.08 113.88) (width 0.2) (layer "B.Cu") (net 6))
 (segment (start 113.04 117.84) (end 113.04 129.57) (width 0.2) (layer "B.Cu") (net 6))
 (segment (start 109.08 113.88) (end 113.04 117.84) (width 0.2) (layer "B.Cu") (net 6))
 (segment (start 145.58 129.57) (end 147.02 128.13) (width 0.2) (layer "B.Cu") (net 6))
 (segment (start 113.04 129.57) (end 145.58 129.57) (width 0.2) (layer "B.Cu") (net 6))
 (segment (start 147.02 128.13) (end 147.02 120.94) (width 0.2) (layer "B.Cu") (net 6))
 (segment (start 131.5 85.23) (end 131.5 93.37) (width 0.2) (layer "F.Cu") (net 15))
 (segment (start 79.5945 88.53025) (end 81.50975 88.53025) (width 0.2) (layer "F.Cu") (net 15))
 (segment (start 82.3 85.25) (end 83.52 84.03) (width 0.2) (layer "F.Cu") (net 15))
 (segment (start 83.52 84.03) (end 130.3 84.03) (width 0.2) (layer "F.Cu") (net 15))
 (segment (start 81.50975 88.53025) (end 82.3 87.74) (width 0.2) (layer "F.Cu") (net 15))
 (segment (start 82.3 87.74) (end 82.3 85.25) (width 0.2) (layer "F.Cu") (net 15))
 (segment (start 130.3 84.03) (end 131.5 85.23) (width 0.2) (layer "F.Cu") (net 15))
 (segment (start 90.98 84.64) (end 117.6 84.64) (width 0.2) (layer "F.Cu") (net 13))
 (segment (start 118.45 98.37) (end 117 98.37) (width 0.2) (layer "F.Cu") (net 13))
 (segment (start 117.6 84.64) (end 119.63 86.67) (width 0.2) (layer "F.Cu") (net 13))
 (segment (start 90.98 89.68) (end 90.98 84.64) (width 0.2) (layer "F.Cu") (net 13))
 (segment (start 89.58975 91.07025) (end 90.98 89.68) (width 0.2) (layer "F.Cu") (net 13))
 (segment (start 79.5945 91.07025) (end 89.58975 91.07025) (width 0.2) (layer "F.Cu") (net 13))
 (segment (start 119.63 97.19) (end 118.45 98.37) (width 0.2) (layer "F.Cu") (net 13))
 (segment (start 119.63 86.67) (end 119.63 97.19) (width 0.2) (layer "F.Cu") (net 13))
 (segment (start 79.5945 93.61025) (end 76.67975 93.61025) (width 0.2) (layer "F.Cu") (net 12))
 (segment (start 76.67975 93.61025) (end 76.56 93.73) (width 0.2) (layer "F.Cu") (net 12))
 (via (at 76.56 93.73) (size 0.6) (drill 0.3) (layers "F.Cu" "B.Cu") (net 12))
 (segment (start 76.56 93.73) (end 77.95 92.34) (width 0.2) (layer "B.Cu") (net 12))
 (segment (start 115.97 92.34) (end 117 93.37) (width 0.2) (layer "B.Cu") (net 12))
 (segment (start 77.95 92.34) (end 115.97 92.34) (width 0.2) (layer "B.Cu") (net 12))
 (segment (start 79.53475 101.29) (end 76.13 101.29) (width 0.2) (layer "F.Cu") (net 1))
 (segment (start 79.5945 101.23025) (end 79.53475 101.29) (width 0.2) (layer "F.Cu") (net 1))
 (via (at 76.13 101.29) (size 0.6) (drill 0.3) (layers "F.Cu" "B.Cu") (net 1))
 (segment (start 76.13 101.29) (end 74.71 101.29) (width 0.2) (layer "B.Cu") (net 1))
 (segment (start 73.13 102.87) (end 73.13 128.68) (width 0.2) (layer "B.Cu") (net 1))
 (segment (start 153.79 128.22) (end 153.79 91.39) (width 0.2) (layer "B.Cu") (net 1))
 (segment (start 73.13 128.68) (end 74.55 130.1) (width 0.2) (layer "B.Cu") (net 1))
 (segment (start 151.91 130.1) (end 153.79 128.22) (width 0.2) (layer "B.Cu") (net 1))
 (segment (start 74.55 130.1) (end 151.91 130.1) (width 0.2) (layer "B.Cu") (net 1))
 (segment (start 145.21 93.37) (end 136.58 93.37) (width 0.2) (layer "B.Cu") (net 1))
 (segment (start 149.07 89.51) (end 145.21 93.37) (width 0.2) (layer "B.Cu") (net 1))
 (segment (start 153.79 91.39) (end 151.91 89.51) (width 0.2) (layer "B.Cu") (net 1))
 (segment (start 151.91 89.51) (end 149.07 89.51) (width 0.2) (layer "B.Cu") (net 1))
 (segment (start 74.71 101.29) (end 73.13 102.87) (width 0.2) (layer "B.Cu") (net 1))
 (segment (start 79.5945 96.15025) (end 79.25475 96.49) (width 0.2) (layer "F.Cu") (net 5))
 (segment (start 79.25475 96.49) (end 77.43 96.49) (width 0.2) (layer "F.Cu") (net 5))
 (segment (start 77.43 96.49) (end 77.35 96.49) (width 0.2) (layer "F.Cu") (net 5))
 (via (at 77.43 96.49) (size 0.6) (drill 0.3) (layers "F.Cu" "B.Cu") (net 5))
 (segment (start 130.23 101.67) (end 139.53 101.67) (width 0.2) (layer "B.Cu") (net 5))
 (segment (start 116.9 101.75) (end 119.41 101.75) (width 0.2) (layer "B.Cu") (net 5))
 (segment (start 111.64 96.49) (end 116.9 101.75) (width 0.2) (layer "B.Cu") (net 5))
 (segment (start 127.11 98.55) (end 130.23 101.67) (width 0.2) (layer "B.Cu") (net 5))
 (segment (start 147.83 93.37) (end 151.08 93.37) (width 0.2) (layer "B.Cu") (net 5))
 (segment (start 77.43 96.49) (end 111.64 96.49) (width 0.2) (layer "B.Cu") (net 5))
 (segment (start 122.61 98.55) (end 127.11 98.55) (width 0.2) (layer "B.Cu") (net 5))
 (segment (start 139.53 101.67) (end 147.83 93.37) (width 0.2) (layer "B.Cu") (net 5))
 (segment (start 119.41 101.75) (end 122.61 98.55) (width 0.2) (layer "B.Cu") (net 5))
 (segment (start 79.5945 98.69025) (end 89.31025 98.69025) (width 0.2) (layer "F.Cu") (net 2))
 (segment (start 94.27 103.65) (end 131.3 103.65) (width 0.2) (layer "F.Cu") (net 2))
 (segment (start 89.31025 98.69025) (end 94.27 103.65) (width 0.2) (layer "F.Cu") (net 2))
 (segment (start 131.3 103.65) (end 136.58 98.37) (width 0.2) (layer "F.Cu") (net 2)))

